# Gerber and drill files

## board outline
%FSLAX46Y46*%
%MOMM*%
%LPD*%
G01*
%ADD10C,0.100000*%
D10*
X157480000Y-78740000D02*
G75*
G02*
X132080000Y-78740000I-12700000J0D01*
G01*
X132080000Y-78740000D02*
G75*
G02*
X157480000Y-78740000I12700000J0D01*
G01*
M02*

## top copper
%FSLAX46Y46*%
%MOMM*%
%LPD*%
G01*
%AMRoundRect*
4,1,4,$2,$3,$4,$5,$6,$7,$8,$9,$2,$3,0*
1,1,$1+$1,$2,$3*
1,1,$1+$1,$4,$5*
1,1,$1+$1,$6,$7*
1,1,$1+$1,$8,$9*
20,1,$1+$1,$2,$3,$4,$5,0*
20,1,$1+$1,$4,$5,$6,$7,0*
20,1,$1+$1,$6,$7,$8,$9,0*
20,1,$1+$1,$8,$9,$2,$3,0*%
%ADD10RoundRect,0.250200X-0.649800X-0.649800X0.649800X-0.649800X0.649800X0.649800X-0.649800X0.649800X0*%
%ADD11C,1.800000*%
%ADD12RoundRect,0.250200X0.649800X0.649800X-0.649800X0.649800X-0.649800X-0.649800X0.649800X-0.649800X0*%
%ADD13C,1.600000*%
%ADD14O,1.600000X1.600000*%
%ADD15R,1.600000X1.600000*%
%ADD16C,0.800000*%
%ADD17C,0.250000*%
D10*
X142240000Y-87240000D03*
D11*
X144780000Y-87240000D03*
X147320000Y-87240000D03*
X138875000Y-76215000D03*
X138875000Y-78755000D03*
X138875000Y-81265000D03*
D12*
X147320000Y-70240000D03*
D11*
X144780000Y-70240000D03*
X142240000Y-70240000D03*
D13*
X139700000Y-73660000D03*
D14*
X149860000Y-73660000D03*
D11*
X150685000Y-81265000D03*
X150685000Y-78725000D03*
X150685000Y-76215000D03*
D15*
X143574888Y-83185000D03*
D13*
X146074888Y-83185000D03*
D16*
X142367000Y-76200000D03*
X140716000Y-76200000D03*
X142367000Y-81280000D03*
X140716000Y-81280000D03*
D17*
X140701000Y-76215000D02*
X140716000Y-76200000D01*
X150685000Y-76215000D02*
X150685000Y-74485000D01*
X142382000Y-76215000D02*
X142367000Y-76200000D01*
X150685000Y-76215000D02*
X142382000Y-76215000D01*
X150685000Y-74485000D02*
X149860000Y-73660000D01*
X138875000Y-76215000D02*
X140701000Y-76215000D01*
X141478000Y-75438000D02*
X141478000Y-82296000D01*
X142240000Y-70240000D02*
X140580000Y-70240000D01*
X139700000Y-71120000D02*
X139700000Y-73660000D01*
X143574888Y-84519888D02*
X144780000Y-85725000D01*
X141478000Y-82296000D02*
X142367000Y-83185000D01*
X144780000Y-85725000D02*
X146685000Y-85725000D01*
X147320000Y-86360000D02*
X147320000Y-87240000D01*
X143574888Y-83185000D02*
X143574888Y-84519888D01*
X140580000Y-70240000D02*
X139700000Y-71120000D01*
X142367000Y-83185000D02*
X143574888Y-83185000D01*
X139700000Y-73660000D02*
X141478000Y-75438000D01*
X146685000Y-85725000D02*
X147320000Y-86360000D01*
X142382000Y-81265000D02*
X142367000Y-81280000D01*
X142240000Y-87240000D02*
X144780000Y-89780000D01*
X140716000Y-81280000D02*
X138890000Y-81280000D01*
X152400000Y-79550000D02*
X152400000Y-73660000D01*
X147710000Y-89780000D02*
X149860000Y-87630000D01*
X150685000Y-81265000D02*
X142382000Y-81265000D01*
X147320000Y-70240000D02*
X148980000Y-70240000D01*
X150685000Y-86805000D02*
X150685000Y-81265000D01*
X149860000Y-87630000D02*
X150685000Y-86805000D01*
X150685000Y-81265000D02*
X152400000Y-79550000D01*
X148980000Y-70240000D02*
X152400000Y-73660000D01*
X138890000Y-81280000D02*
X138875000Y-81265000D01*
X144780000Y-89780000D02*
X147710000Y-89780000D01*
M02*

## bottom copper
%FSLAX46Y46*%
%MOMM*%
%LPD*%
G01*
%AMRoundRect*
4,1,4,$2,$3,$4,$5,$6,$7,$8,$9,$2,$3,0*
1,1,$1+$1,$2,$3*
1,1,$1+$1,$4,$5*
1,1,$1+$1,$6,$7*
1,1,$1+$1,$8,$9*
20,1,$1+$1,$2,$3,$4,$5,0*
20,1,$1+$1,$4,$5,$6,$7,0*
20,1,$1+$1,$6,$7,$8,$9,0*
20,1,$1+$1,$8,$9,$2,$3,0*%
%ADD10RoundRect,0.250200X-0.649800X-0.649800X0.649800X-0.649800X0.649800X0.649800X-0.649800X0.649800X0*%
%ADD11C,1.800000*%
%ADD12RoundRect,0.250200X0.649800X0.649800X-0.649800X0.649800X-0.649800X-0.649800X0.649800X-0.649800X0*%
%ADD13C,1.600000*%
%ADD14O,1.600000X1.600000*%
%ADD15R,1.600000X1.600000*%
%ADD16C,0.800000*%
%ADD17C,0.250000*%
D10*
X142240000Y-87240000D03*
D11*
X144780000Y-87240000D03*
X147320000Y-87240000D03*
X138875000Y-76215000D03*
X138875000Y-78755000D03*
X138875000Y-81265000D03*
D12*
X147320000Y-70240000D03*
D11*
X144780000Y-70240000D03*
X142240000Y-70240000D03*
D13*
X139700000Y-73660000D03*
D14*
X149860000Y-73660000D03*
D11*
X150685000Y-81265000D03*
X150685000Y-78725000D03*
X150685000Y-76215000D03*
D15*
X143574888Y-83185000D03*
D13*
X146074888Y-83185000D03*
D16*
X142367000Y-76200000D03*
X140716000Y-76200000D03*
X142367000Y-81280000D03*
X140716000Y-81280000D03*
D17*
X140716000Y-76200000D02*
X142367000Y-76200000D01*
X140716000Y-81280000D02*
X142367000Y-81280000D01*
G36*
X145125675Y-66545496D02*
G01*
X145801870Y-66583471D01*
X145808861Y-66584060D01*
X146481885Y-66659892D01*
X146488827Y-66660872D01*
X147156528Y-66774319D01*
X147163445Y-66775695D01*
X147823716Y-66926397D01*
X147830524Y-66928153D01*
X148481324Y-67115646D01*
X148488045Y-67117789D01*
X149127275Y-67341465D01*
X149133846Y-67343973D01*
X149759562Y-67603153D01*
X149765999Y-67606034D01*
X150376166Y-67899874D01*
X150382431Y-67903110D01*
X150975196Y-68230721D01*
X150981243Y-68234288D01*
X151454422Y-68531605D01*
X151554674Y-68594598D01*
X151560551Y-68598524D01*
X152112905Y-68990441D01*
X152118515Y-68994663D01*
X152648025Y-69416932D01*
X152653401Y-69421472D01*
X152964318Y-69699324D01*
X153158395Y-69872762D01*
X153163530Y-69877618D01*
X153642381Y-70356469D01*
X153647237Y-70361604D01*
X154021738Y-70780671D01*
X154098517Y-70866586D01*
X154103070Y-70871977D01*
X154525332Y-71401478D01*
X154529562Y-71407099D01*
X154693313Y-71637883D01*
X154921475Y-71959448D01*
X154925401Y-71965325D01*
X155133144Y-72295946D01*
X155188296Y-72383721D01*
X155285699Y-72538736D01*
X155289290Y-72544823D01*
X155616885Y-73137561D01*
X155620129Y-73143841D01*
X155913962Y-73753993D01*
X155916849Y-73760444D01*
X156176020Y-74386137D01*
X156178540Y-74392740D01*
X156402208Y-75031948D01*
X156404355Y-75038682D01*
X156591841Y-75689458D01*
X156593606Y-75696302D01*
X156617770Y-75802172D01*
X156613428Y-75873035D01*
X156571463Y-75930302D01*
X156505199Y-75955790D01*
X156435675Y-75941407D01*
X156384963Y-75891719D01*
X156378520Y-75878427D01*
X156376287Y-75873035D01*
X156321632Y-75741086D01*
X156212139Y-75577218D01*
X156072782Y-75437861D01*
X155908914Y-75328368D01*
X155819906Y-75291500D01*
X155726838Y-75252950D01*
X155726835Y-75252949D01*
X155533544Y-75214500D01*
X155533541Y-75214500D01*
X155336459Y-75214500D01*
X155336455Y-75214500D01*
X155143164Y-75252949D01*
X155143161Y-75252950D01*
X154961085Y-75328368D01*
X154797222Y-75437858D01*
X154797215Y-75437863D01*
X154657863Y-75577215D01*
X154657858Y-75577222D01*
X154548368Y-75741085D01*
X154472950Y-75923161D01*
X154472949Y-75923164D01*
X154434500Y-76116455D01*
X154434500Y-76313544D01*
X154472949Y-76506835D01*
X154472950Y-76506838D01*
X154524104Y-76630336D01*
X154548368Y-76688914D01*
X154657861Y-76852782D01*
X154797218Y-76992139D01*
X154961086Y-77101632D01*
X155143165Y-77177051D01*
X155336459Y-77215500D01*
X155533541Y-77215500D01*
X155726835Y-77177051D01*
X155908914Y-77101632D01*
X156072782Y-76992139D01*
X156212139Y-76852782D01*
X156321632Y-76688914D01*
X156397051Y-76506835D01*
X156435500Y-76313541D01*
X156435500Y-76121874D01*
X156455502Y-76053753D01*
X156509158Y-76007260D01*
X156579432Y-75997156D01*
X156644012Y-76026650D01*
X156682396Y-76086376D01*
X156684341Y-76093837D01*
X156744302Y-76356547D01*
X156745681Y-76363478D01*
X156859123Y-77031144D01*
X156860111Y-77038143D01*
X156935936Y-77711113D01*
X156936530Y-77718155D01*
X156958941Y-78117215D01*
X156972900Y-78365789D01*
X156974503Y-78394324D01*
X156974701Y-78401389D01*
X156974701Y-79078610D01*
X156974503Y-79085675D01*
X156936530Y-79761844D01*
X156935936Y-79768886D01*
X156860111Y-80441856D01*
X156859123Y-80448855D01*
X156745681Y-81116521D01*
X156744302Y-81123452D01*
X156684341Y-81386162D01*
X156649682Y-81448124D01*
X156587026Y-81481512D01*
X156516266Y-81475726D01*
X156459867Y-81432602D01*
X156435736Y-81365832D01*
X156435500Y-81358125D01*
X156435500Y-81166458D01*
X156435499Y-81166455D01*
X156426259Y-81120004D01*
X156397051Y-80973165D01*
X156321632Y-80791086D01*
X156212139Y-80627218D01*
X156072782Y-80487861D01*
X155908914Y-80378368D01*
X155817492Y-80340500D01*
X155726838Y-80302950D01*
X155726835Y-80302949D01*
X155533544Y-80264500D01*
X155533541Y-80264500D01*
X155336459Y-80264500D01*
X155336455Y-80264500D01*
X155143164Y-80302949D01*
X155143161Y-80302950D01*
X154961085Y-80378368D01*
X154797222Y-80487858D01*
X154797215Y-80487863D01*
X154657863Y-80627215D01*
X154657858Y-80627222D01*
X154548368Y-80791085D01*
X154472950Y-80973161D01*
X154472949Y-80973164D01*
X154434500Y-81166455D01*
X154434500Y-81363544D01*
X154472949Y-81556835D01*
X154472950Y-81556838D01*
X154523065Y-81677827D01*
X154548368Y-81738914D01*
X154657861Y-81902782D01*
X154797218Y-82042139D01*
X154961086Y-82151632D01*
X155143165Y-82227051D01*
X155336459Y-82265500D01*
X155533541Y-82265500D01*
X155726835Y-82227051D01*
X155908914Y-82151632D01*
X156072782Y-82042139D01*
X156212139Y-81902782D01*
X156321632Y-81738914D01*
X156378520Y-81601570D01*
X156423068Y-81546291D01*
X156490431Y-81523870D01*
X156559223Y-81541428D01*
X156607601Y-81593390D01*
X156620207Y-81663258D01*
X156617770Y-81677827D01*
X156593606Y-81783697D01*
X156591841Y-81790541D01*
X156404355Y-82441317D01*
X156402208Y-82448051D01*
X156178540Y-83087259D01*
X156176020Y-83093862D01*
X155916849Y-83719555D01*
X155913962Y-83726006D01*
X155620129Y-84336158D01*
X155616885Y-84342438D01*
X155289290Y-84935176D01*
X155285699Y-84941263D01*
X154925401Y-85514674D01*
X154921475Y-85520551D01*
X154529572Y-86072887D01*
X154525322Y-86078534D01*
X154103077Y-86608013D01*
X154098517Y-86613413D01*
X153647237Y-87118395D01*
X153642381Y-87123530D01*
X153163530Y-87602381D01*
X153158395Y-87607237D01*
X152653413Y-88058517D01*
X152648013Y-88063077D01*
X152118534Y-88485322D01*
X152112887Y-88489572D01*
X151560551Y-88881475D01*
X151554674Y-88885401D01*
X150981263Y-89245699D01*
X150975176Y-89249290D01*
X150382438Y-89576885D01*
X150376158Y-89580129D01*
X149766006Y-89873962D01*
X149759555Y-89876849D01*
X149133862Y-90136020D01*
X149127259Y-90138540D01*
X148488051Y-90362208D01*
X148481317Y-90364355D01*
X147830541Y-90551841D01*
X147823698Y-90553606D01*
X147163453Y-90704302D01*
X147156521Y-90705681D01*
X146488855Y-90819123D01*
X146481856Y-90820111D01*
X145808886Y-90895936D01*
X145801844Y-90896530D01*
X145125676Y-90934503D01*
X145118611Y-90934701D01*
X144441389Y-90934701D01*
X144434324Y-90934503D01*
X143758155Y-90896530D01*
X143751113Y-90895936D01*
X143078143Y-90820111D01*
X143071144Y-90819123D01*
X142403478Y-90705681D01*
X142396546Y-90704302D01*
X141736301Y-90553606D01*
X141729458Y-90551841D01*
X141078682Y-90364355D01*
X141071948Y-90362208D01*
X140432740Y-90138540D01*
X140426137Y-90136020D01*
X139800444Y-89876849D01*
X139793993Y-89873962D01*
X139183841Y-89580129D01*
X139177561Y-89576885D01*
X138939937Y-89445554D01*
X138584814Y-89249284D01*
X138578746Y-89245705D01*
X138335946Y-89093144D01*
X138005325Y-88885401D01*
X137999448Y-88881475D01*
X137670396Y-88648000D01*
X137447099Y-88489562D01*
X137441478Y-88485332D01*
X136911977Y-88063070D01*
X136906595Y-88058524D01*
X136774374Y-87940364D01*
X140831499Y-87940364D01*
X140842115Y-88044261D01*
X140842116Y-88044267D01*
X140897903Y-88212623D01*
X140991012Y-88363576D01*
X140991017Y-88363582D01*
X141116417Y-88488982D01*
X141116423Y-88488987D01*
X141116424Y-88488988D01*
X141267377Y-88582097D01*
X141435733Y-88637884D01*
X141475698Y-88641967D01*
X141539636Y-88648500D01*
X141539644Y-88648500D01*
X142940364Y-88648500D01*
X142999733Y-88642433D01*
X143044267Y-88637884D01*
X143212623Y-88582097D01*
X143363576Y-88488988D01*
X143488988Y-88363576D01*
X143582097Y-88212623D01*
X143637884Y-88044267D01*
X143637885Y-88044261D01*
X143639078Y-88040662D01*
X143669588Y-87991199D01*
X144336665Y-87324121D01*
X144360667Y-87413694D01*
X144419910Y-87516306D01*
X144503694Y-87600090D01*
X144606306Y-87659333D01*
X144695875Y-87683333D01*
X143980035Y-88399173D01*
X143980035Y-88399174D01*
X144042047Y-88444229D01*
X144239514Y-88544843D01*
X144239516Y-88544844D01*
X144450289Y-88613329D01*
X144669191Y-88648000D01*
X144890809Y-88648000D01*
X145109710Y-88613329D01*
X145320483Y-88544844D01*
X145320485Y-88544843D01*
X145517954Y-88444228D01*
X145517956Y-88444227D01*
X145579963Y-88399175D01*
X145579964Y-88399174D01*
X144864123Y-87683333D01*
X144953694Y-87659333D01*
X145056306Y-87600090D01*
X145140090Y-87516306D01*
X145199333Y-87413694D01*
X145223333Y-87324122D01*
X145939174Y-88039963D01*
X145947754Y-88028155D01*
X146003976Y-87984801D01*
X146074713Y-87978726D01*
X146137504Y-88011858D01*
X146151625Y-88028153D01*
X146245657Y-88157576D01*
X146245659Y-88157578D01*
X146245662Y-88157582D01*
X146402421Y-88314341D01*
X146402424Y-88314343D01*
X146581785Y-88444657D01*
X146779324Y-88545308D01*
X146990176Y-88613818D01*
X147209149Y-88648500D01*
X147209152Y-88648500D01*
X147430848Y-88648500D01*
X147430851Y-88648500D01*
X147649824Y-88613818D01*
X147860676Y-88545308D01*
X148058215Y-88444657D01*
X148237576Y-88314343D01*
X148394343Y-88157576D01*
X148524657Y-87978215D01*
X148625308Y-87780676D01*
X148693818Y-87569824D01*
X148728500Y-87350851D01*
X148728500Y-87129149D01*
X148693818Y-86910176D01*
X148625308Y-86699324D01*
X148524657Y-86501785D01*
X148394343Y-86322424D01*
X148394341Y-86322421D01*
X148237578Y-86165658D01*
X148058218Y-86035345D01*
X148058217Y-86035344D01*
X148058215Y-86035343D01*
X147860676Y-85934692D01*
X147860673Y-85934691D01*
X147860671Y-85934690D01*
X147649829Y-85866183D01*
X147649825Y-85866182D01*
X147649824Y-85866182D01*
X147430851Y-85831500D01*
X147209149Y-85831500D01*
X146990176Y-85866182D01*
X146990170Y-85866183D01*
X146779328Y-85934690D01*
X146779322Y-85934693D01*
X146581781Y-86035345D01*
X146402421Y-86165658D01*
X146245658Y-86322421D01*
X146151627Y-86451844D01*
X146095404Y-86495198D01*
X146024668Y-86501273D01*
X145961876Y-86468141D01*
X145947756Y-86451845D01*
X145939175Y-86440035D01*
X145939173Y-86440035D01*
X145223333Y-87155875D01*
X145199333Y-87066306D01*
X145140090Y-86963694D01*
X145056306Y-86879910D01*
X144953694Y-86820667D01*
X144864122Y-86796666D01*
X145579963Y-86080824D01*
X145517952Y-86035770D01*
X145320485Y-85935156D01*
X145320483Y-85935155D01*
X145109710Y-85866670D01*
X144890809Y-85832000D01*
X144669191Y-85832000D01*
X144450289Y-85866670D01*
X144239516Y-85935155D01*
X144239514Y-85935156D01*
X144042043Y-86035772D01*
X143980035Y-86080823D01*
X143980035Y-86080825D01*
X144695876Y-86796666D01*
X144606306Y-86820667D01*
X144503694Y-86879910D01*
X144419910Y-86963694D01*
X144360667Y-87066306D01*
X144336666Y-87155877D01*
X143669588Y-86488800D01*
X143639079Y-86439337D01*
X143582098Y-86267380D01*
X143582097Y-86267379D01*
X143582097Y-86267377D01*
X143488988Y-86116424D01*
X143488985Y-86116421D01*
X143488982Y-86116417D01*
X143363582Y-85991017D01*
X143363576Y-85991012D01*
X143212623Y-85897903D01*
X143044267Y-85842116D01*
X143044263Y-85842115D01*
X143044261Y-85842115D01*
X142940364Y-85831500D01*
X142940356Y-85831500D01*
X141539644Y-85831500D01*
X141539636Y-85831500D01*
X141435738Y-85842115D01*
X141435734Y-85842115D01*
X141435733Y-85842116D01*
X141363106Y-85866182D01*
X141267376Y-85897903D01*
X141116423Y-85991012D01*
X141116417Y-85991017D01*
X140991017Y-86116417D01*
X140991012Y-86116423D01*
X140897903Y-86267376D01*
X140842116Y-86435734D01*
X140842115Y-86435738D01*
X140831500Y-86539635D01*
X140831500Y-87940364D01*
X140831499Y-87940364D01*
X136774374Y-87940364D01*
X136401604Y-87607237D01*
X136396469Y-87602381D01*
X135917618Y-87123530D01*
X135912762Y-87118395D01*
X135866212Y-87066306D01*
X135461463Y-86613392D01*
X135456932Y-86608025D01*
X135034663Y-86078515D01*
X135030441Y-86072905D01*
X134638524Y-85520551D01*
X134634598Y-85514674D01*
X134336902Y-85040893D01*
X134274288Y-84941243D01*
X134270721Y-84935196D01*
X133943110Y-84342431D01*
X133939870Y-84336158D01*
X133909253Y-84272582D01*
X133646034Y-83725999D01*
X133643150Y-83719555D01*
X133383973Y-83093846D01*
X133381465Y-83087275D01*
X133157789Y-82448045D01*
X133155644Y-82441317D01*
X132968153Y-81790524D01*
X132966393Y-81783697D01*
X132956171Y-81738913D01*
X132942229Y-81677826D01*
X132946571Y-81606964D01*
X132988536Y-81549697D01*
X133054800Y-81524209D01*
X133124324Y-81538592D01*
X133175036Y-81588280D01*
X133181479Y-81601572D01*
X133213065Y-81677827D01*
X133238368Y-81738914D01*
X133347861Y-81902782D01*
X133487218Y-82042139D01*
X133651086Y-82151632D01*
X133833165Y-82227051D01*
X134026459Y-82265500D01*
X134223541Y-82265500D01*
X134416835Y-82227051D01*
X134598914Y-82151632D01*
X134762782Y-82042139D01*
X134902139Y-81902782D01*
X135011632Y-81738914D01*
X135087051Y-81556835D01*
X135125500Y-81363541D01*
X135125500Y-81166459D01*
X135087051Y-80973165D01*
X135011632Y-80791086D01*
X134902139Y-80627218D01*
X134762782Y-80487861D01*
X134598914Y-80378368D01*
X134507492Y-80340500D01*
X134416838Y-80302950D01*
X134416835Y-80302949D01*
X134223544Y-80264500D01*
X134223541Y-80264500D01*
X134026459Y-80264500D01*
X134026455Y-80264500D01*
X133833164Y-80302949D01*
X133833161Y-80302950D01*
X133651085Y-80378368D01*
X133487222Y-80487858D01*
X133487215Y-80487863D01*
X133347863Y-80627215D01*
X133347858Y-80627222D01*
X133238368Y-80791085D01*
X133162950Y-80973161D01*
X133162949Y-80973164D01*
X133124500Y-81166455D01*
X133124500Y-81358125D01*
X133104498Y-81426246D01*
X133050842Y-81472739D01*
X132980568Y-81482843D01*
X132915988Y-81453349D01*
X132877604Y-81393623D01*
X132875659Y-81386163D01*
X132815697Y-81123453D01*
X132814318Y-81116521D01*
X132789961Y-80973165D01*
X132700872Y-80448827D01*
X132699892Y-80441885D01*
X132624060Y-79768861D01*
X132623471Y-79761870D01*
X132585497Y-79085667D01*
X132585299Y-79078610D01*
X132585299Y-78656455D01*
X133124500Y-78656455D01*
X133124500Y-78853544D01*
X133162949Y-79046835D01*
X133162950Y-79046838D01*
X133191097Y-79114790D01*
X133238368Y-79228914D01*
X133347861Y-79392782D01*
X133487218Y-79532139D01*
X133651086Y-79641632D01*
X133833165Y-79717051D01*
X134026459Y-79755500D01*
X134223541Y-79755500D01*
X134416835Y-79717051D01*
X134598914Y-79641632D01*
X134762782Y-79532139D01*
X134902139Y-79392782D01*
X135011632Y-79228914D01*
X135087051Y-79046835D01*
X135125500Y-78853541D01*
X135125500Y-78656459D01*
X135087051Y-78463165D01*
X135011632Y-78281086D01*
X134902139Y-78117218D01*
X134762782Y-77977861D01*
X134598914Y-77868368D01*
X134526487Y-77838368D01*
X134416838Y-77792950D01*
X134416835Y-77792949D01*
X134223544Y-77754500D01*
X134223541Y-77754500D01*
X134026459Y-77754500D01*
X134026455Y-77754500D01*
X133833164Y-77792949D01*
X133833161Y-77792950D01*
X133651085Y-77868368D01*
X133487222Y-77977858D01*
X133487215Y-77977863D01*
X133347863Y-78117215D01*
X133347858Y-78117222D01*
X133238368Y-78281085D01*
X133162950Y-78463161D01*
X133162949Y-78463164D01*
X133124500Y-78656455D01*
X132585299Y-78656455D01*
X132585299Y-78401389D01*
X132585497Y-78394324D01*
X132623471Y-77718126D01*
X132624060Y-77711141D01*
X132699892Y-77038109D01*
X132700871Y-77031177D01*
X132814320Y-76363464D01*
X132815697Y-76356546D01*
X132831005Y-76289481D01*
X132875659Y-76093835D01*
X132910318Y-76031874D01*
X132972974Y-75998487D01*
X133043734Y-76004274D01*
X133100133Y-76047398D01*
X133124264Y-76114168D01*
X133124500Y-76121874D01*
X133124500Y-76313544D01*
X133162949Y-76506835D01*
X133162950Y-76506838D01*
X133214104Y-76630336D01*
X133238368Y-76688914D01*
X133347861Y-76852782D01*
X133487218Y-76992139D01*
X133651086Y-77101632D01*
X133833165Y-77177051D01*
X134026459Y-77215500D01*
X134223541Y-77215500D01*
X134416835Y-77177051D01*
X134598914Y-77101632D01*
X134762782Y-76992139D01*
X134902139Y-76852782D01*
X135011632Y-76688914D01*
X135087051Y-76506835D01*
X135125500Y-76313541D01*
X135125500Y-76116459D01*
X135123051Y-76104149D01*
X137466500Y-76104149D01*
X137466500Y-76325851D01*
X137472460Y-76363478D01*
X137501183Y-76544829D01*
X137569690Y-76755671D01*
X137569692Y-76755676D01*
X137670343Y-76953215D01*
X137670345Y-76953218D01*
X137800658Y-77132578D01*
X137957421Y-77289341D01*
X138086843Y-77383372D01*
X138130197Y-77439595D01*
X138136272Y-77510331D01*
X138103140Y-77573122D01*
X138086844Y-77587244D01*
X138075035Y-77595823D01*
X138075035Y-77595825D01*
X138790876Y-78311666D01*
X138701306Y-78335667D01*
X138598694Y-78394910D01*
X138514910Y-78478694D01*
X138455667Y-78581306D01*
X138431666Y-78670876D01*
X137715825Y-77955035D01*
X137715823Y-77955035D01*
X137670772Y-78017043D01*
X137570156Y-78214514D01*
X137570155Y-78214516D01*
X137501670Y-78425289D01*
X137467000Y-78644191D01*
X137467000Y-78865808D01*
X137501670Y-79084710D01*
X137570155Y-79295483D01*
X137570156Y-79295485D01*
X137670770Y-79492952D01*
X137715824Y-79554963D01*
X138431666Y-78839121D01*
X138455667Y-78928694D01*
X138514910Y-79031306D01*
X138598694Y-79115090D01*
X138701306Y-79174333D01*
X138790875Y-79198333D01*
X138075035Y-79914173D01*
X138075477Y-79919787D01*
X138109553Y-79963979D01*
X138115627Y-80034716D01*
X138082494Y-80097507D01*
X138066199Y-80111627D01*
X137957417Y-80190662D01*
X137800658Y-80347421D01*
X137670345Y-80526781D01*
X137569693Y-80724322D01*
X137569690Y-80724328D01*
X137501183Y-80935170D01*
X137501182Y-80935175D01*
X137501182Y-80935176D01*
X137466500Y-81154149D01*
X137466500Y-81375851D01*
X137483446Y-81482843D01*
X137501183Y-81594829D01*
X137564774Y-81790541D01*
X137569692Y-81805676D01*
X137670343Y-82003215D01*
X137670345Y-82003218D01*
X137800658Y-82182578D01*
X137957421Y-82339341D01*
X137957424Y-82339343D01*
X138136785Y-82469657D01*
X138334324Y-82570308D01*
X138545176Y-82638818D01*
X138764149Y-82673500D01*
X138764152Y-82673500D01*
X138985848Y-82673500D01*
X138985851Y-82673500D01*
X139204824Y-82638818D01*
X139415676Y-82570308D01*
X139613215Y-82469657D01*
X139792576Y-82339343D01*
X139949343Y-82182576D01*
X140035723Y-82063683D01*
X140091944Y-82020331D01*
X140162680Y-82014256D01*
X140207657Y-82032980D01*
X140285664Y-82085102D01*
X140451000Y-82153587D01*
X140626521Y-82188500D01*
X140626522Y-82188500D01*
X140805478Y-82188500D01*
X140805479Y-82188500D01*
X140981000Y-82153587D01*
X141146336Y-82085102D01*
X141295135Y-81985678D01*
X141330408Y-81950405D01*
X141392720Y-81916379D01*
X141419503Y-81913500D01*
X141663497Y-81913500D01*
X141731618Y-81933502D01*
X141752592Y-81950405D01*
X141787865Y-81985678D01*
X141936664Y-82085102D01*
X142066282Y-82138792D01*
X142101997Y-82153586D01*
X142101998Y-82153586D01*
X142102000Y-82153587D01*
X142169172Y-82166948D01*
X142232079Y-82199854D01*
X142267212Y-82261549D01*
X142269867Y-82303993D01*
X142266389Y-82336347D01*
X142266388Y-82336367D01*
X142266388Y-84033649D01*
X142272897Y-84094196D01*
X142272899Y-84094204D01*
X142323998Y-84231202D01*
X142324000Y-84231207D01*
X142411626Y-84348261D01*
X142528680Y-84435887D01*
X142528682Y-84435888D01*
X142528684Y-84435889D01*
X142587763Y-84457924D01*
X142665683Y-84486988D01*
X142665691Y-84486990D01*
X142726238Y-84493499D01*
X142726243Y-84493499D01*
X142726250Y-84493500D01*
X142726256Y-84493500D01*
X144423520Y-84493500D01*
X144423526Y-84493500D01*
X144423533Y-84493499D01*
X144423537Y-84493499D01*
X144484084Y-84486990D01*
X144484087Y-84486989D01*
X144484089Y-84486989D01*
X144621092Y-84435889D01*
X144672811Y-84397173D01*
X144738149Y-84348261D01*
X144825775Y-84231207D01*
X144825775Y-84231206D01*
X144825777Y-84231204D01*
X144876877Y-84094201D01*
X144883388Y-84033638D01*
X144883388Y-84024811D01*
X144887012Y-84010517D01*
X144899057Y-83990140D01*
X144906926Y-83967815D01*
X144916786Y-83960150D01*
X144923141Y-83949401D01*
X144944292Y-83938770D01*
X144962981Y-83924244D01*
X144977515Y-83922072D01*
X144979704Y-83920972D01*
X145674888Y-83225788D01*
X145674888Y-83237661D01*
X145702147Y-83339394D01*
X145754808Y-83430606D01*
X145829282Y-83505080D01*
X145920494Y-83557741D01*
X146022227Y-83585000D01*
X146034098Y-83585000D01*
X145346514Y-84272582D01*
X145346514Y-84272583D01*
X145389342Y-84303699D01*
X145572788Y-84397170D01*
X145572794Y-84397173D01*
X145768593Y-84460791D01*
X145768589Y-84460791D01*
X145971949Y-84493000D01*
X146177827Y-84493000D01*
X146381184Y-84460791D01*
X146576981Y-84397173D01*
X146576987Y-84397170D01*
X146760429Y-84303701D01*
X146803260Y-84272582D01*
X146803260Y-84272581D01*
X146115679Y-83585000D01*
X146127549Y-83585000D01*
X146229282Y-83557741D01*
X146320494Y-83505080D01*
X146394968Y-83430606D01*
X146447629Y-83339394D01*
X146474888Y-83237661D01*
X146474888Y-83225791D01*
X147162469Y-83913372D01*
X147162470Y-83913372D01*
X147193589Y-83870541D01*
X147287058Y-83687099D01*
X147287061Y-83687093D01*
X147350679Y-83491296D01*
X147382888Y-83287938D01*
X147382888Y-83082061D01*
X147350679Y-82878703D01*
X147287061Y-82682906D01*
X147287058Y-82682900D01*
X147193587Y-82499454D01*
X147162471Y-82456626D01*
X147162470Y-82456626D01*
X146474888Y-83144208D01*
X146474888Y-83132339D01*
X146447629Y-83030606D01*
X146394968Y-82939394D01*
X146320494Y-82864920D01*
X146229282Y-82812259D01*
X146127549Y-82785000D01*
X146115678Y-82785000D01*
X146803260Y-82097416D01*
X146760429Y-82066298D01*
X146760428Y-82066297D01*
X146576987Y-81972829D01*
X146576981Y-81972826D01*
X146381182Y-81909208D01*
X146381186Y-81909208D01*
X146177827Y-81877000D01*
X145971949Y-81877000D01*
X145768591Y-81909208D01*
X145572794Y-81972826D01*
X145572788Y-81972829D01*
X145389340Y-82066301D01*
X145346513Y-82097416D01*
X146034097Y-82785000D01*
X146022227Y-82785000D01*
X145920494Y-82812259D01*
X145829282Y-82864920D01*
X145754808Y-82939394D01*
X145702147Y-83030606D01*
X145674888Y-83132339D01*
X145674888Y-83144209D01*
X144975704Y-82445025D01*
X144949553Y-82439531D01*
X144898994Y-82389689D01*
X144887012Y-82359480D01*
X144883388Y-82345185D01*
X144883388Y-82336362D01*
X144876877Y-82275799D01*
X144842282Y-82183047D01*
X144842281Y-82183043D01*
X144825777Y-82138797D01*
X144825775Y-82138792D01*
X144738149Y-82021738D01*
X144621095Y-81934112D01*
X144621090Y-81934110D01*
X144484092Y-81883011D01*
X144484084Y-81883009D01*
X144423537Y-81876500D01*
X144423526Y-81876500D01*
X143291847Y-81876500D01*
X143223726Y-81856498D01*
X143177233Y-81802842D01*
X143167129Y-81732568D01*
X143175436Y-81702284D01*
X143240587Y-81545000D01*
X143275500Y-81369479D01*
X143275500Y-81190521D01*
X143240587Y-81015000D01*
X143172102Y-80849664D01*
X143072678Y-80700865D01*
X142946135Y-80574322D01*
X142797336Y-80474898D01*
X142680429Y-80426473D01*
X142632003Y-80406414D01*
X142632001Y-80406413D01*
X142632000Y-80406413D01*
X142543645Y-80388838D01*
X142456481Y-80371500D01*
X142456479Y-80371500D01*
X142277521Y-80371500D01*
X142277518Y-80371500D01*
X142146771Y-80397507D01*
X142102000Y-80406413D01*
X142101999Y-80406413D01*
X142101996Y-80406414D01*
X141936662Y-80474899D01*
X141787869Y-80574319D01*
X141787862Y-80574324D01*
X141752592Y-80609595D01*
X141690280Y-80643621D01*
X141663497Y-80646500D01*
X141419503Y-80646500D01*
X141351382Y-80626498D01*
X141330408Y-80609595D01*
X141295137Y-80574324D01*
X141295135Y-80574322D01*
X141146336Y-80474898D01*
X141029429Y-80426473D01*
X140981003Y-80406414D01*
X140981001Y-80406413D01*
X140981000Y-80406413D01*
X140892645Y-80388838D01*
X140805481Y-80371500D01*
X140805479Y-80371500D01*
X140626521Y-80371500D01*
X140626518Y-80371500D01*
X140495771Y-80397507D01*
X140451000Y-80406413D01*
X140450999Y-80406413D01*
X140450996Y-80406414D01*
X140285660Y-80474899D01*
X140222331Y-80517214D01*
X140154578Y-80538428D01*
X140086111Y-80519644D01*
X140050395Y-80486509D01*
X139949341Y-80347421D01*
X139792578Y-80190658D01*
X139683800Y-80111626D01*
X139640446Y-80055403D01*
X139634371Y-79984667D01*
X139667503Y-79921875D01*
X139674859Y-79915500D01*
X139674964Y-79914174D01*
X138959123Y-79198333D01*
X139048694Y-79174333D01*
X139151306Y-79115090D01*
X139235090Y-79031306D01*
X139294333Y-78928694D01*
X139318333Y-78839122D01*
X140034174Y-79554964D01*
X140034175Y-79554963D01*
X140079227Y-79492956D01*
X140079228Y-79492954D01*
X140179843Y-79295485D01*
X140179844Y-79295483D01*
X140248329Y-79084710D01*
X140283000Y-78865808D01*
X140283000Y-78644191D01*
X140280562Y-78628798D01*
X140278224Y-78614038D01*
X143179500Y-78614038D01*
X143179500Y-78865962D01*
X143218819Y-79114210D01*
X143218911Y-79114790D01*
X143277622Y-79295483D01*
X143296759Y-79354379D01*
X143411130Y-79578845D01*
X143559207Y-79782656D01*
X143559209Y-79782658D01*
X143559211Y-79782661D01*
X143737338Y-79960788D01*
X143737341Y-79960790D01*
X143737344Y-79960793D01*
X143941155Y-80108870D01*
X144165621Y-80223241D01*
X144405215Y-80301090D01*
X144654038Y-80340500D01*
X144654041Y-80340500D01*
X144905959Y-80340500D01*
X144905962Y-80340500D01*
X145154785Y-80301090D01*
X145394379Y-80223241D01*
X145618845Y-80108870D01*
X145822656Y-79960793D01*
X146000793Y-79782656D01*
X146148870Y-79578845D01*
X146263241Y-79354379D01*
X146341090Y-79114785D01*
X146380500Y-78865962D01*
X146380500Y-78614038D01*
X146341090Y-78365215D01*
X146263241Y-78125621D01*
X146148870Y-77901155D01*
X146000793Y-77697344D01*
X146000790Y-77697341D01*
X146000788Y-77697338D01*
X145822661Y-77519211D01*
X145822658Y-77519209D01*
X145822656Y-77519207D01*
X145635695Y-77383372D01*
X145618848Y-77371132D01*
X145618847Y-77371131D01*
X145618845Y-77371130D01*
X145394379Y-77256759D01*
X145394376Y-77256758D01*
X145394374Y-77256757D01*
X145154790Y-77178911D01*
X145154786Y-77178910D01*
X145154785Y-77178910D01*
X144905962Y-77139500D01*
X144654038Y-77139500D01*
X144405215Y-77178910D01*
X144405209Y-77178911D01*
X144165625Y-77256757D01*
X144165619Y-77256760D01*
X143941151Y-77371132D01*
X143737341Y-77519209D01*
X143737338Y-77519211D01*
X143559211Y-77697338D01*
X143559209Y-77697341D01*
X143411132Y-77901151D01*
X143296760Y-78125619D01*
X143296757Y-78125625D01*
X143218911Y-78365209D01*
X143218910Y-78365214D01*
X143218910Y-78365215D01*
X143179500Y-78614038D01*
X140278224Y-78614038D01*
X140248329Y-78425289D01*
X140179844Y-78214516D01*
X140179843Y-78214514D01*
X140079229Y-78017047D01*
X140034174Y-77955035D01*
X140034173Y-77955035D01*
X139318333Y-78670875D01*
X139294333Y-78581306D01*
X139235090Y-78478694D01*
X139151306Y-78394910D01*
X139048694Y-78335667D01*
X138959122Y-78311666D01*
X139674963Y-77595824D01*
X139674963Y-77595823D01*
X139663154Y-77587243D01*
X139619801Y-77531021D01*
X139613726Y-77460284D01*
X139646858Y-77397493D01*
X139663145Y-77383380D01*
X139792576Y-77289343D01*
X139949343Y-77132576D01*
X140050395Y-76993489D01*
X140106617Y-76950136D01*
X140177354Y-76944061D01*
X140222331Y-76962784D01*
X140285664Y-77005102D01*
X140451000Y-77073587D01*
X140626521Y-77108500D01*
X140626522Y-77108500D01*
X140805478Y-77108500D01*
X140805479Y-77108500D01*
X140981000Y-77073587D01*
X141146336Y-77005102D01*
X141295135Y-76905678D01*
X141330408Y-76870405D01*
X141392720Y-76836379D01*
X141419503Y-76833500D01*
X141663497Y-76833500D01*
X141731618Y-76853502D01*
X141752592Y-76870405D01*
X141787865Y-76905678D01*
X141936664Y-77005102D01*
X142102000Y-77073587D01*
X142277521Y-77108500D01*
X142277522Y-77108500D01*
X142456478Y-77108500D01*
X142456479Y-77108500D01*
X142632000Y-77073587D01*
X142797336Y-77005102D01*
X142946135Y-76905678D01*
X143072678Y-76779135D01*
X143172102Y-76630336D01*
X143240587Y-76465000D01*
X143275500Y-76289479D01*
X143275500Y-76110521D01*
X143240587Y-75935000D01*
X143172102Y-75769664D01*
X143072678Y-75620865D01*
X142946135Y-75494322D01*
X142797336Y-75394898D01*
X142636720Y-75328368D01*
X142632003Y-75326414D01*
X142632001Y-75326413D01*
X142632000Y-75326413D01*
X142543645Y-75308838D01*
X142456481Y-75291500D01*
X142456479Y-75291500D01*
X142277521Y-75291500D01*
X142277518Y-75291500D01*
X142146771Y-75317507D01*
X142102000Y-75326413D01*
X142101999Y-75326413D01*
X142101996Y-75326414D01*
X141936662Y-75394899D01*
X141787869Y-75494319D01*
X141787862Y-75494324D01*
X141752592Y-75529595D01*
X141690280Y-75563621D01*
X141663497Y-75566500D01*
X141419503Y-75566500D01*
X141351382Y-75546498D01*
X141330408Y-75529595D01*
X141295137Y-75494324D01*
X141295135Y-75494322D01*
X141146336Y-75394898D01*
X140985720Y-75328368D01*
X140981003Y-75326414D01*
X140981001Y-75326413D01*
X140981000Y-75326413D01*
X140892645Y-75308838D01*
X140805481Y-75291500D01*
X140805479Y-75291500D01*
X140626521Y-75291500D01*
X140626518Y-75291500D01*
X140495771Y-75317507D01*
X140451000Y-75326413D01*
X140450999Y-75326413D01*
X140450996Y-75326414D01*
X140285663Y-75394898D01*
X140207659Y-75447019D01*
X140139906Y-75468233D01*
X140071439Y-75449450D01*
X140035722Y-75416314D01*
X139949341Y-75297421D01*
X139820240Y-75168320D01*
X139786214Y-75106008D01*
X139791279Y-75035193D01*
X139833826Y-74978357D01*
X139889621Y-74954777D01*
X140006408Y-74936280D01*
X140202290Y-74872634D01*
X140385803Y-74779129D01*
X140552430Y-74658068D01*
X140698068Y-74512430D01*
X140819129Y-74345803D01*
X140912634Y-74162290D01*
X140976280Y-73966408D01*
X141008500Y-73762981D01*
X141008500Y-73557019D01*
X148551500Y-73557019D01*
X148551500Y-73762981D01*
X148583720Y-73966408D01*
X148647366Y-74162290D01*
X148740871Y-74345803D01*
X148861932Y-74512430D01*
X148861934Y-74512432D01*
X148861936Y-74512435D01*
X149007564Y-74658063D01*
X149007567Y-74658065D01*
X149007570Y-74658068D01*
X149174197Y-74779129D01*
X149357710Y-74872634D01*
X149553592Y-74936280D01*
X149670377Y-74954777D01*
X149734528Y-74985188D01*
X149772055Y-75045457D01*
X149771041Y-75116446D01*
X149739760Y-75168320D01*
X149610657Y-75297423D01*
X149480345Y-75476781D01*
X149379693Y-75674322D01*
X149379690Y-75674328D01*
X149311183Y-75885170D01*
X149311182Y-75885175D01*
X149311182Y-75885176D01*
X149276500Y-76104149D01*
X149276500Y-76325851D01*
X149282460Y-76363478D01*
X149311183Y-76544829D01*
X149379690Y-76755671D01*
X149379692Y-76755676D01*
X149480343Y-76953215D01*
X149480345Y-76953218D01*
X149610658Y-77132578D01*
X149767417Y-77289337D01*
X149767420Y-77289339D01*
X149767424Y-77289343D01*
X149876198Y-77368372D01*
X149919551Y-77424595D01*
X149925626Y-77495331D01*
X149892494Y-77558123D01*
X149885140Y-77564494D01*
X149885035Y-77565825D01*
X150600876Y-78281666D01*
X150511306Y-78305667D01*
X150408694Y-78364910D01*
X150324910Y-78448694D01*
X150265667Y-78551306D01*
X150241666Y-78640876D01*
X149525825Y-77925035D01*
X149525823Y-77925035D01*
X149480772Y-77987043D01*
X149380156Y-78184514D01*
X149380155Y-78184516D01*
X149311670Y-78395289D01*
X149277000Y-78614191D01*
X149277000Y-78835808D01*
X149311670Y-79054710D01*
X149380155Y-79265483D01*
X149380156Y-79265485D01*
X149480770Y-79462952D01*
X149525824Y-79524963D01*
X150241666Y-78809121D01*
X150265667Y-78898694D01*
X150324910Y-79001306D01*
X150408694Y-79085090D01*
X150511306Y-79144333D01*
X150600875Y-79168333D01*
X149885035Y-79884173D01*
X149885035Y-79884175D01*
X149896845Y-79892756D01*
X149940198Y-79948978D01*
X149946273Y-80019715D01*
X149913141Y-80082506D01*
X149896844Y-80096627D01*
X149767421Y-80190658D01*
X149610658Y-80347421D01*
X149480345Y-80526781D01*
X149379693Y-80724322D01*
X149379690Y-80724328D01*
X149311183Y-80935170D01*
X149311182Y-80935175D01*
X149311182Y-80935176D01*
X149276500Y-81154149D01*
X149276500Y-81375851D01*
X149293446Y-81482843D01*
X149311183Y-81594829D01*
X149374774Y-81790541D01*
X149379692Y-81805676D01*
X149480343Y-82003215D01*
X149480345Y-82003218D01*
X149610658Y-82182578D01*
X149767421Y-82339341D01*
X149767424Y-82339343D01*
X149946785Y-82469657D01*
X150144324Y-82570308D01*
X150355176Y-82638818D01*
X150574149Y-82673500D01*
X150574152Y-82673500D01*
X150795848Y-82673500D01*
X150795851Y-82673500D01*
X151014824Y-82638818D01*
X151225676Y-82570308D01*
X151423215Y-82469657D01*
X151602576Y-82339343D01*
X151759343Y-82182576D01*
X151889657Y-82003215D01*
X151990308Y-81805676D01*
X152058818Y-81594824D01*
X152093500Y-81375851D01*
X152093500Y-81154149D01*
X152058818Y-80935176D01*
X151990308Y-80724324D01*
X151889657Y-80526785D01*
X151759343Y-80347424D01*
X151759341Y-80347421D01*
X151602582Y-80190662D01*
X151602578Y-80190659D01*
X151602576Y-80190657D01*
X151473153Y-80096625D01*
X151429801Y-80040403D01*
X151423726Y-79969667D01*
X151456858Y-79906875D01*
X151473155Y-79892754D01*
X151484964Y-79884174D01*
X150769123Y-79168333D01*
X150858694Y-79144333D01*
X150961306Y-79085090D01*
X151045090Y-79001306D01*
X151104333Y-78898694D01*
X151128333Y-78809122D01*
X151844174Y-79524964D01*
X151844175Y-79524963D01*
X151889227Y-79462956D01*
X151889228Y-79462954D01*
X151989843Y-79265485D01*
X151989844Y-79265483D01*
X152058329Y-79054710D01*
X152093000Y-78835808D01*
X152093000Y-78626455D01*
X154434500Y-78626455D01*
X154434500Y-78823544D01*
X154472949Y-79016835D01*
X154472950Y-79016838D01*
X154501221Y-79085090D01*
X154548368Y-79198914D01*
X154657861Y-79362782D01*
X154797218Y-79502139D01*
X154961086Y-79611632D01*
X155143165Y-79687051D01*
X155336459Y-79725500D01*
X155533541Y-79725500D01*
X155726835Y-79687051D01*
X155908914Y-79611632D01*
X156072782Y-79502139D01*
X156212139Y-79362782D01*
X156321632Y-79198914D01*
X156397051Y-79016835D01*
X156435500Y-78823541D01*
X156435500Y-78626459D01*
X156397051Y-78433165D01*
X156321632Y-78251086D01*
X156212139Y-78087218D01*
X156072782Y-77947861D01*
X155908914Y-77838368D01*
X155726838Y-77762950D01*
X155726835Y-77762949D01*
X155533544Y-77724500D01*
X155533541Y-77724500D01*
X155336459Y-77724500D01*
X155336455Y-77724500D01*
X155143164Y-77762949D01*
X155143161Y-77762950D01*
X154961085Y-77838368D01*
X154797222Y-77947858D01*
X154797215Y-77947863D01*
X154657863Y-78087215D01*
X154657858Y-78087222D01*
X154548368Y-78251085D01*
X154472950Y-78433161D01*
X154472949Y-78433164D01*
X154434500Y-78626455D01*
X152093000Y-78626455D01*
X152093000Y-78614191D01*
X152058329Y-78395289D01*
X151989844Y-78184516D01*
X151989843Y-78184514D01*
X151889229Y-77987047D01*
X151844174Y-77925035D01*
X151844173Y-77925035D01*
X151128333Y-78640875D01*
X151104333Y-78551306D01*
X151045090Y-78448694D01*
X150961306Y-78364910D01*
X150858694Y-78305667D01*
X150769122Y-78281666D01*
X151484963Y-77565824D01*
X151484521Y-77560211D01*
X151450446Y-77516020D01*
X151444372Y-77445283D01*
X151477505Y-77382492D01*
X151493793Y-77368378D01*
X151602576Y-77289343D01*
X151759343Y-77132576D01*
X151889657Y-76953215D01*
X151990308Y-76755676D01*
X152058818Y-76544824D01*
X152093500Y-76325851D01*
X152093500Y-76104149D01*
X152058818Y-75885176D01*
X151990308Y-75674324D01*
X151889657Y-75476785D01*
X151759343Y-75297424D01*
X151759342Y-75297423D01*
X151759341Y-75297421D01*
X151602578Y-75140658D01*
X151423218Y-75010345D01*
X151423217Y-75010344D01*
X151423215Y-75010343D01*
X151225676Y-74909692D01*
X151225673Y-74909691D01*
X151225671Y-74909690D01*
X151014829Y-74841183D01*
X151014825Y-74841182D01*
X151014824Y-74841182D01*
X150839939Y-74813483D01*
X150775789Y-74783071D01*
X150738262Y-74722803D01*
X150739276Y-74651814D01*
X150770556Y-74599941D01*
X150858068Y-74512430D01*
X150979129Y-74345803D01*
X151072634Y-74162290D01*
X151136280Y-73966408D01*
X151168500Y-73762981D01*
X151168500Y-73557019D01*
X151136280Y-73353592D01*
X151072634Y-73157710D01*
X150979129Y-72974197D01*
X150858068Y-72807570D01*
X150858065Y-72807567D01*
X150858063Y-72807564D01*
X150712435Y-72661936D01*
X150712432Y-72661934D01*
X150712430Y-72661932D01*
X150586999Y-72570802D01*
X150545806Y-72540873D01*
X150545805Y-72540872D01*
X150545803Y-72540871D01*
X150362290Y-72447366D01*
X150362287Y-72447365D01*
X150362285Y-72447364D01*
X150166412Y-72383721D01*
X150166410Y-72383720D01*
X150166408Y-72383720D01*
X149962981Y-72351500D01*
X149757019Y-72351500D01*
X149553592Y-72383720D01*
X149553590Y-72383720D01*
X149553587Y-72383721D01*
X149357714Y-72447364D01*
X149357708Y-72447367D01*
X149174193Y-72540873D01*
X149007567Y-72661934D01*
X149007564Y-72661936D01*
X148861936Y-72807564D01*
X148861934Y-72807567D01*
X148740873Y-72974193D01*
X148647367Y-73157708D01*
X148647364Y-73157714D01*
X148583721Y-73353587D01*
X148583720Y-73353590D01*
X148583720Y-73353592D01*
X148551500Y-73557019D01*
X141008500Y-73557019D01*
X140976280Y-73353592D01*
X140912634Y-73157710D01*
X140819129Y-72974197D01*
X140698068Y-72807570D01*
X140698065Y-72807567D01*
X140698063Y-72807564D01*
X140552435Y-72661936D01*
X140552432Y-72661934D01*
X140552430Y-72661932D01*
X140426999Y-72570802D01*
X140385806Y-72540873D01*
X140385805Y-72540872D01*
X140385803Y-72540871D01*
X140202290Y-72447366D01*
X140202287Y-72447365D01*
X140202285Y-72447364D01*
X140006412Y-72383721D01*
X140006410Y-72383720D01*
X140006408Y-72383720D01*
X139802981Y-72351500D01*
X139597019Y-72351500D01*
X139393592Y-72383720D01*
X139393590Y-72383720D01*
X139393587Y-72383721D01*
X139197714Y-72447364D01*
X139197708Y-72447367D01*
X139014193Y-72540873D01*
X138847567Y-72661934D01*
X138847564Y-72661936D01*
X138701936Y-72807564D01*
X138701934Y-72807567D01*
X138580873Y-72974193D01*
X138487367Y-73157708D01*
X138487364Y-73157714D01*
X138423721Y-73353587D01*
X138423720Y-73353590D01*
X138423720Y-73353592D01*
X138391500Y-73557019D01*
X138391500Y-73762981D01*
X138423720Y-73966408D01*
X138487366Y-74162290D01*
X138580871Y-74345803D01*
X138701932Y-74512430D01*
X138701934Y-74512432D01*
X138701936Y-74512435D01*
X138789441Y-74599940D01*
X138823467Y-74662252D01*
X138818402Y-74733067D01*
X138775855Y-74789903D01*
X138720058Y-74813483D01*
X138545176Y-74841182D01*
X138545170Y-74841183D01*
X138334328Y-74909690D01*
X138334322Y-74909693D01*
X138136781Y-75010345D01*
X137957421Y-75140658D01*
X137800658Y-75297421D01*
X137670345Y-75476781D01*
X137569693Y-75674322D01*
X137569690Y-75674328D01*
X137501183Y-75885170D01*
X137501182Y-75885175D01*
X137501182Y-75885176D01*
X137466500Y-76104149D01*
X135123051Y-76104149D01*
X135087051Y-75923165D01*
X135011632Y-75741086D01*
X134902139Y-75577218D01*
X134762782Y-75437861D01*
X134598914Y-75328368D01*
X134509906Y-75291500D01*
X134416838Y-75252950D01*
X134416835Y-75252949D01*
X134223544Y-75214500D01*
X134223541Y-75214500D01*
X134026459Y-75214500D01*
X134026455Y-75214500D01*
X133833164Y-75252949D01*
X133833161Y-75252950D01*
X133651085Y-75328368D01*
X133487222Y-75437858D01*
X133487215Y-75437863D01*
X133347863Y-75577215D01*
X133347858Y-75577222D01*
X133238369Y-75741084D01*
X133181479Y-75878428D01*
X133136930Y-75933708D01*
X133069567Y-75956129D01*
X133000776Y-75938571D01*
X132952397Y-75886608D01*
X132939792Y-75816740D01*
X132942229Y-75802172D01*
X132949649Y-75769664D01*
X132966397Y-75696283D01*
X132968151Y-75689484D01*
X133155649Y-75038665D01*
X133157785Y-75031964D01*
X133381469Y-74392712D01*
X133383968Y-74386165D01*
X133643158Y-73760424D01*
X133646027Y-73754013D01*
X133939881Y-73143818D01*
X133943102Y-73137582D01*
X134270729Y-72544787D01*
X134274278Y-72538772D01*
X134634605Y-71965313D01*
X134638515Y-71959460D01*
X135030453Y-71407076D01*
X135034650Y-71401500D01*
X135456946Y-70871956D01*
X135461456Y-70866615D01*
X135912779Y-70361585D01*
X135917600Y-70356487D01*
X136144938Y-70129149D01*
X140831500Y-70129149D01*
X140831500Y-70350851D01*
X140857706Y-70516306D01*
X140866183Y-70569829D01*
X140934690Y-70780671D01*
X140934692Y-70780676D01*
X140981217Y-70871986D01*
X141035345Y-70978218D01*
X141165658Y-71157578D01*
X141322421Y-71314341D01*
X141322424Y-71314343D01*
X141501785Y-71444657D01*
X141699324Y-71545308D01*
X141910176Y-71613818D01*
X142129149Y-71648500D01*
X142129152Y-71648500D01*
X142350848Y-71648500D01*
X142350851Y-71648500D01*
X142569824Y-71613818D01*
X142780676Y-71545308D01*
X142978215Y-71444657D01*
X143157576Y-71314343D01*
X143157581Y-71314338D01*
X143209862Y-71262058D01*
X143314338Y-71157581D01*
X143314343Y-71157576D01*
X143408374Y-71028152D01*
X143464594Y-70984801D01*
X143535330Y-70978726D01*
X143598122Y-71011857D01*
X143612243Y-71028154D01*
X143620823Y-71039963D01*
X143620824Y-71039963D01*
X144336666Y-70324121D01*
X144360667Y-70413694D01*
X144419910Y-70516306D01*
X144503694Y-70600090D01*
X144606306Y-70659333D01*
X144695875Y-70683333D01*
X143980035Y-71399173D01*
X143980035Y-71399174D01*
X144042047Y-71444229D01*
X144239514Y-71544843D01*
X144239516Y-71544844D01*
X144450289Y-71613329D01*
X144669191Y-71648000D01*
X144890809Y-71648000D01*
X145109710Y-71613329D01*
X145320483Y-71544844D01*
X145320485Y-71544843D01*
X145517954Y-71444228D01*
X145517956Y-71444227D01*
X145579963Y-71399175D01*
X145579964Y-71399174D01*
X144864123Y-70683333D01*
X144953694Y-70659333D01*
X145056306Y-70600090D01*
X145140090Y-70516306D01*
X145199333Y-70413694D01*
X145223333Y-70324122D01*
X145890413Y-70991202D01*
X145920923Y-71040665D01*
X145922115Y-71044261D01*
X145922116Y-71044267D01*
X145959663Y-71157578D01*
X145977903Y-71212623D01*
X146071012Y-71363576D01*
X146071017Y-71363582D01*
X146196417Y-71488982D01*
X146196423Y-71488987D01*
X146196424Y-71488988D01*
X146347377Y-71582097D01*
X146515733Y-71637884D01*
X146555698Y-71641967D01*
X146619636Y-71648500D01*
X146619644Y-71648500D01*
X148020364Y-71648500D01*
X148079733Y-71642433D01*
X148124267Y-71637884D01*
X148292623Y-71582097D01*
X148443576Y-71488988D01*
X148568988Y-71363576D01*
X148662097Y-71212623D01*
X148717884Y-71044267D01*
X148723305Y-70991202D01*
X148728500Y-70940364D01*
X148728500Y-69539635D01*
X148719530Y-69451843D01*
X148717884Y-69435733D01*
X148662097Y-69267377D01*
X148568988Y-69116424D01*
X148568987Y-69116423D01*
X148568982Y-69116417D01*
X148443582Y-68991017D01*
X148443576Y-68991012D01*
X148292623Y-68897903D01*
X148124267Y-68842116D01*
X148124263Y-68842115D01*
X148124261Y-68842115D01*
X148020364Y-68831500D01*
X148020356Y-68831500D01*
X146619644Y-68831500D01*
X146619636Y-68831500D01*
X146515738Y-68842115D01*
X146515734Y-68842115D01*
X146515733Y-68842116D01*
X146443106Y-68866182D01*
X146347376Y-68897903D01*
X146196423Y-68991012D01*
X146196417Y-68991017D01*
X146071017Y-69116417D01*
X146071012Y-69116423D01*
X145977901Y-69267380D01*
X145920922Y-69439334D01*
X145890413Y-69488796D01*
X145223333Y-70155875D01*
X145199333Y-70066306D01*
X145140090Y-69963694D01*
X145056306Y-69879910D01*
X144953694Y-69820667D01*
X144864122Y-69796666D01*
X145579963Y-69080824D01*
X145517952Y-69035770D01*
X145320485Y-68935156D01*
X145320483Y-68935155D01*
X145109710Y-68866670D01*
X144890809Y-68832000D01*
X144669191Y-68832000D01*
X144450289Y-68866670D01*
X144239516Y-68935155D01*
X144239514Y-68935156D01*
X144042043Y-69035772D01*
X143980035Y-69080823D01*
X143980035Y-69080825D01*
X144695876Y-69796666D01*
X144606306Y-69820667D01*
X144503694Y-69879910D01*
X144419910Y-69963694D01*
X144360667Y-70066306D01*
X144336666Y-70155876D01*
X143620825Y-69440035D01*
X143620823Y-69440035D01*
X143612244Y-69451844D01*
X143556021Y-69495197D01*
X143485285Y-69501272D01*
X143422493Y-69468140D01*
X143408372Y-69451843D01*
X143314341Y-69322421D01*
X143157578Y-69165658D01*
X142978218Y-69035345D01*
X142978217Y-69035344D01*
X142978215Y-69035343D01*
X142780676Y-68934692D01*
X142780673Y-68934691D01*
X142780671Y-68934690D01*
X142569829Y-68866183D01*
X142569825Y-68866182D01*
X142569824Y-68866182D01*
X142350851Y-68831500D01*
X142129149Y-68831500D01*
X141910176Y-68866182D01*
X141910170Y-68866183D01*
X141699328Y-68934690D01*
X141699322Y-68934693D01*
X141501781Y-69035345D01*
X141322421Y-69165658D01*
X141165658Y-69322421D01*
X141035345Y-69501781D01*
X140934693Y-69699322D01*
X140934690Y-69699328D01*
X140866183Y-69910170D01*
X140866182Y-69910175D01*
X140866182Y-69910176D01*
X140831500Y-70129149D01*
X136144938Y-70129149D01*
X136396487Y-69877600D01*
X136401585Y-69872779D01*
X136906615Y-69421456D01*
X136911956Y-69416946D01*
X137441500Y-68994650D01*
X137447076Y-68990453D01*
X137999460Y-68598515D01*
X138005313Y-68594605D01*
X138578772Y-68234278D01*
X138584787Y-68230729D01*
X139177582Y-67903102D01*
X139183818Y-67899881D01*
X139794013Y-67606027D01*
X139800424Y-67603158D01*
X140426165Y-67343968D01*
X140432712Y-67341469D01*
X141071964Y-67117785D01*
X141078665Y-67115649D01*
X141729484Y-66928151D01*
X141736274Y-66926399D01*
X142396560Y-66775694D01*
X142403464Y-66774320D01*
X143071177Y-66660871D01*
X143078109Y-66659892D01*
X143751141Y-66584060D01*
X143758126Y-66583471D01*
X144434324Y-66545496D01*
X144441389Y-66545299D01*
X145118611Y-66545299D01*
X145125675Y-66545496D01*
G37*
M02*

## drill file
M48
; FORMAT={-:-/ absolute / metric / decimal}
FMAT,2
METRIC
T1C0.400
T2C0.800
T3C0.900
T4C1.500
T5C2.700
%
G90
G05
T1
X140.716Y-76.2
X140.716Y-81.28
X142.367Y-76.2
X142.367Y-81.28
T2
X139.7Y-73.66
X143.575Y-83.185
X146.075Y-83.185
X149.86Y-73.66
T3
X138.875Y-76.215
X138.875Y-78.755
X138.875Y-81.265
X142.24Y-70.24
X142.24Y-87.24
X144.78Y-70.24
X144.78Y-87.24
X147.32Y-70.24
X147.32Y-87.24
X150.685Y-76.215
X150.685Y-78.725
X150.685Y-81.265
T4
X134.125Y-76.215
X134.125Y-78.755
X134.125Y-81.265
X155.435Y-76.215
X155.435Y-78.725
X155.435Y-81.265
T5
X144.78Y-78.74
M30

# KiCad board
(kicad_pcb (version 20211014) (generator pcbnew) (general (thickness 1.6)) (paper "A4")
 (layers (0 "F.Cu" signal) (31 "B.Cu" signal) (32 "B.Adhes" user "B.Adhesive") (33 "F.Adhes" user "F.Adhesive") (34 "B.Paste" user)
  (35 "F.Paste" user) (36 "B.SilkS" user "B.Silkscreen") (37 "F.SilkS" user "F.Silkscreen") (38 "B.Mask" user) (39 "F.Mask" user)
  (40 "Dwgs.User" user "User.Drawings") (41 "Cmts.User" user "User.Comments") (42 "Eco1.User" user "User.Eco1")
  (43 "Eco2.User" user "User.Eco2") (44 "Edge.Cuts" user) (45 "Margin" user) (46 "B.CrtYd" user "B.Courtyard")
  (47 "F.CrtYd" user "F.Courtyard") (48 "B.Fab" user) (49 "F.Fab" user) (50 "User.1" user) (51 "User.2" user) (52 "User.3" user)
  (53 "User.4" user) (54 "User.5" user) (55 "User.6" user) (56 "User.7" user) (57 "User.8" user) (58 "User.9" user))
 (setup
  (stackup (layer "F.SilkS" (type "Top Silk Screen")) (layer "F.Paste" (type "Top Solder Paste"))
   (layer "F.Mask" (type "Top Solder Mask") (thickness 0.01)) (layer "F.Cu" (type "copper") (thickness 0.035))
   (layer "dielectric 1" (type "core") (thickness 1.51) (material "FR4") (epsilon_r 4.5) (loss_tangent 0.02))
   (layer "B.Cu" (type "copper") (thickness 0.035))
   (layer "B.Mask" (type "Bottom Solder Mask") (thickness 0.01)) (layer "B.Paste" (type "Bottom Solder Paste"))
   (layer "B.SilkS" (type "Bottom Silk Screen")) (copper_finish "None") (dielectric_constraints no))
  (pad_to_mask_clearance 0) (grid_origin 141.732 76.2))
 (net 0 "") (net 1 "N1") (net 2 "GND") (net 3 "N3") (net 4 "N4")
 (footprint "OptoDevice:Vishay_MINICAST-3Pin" (layer "F.Cu") (at 142.24 87.24)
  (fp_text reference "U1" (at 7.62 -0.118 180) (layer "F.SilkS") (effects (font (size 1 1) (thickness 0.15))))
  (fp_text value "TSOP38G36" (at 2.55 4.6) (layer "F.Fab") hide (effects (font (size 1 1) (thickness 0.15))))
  (pad "1" thru_hole roundrect (at 0 0) (size 1.8 1.8) (drill 0.9) (layers *.Cu *.Mask) (roundrect_rratio 0.139) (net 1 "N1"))
  (pad "2" thru_hole circle (at 2.54 0) (size 1.8 1.8) (drill 0.9) (layers *.Cu *.Mask) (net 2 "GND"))
  (pad "3" thru_hole circle (at 5.08 0) (size 1.8 1.8) (drill 0.9) (layers *.Cu *.Mask) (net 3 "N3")))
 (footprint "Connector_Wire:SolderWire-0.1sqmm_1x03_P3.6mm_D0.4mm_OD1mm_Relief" (layer "F.Cu") (at 138.875 75.155 -90)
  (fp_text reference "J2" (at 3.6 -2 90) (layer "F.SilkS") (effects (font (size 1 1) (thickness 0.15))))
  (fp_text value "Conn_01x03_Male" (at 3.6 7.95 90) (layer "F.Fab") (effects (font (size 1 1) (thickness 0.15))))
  (pad "" np_thru_hole circle (at 6.11 4.75 270) (size 1.5 1.5) (drill 1.5) (layers *.Cu *.Mask))
  (pad "" np_thru_hole circle (at 3.6 4.75 270) (size 1.5 1.5) (drill 1.5) (layers *.Cu *.Mask))
  (pad "" np_thru_hole circle (at 1.06 4.75 270) (size 1.5 1.5) (drill 1.5) (layers *.Cu *.Mask))
  (pad "1" thru_hole circle (at 1.06 0 270) (size 1.8 1.8) (drill 0.9) (layers *.Cu *.Mask) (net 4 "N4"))
  (pad "2" thru_hole circle (at 3.6 0 270) (size 1.8 1.8) (drill 0.9) (layers *.Cu *.Mask) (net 2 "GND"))
  (pad "3" thru_hole circle (at 6.11 0 270) (size 1.8 1.8) (drill 0.9) (layers *.Cu *.Mask) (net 1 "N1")))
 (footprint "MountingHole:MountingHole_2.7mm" (layer "F.Cu") (at 144.78 78.74)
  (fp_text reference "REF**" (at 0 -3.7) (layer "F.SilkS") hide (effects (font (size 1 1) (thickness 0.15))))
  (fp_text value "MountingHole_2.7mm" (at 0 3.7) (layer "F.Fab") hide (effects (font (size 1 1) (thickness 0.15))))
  (pad "" np_thru_hole circle (at 0 0) (size 2.7 2.7) (drill 2.7) (layers *.Cu *.Mask)))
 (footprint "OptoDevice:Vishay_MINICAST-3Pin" (layer "F.Cu") (at 147.32 70.24 180)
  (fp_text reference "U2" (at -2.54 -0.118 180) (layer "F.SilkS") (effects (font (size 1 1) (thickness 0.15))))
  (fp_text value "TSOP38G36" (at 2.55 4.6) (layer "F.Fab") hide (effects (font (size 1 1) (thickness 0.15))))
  (pad "1" thru_hole roundrect (at 0 0 180) (size 1.8 1.8) (drill 0.9) (layers *.Cu *.Mask) (roundrect_rratio 0.139) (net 1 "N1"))
  (pad "2" thru_hole circle (at 2.54 0 180) (size 1.8 1.8) (drill 0.9) (layers *.Cu *.Mask) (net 2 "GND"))
  (pad "3" thru_hole circle (at 5.08 0 180) (size 1.8 1.8) (drill 0.9) (layers *.Cu *.Mask) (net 3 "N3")))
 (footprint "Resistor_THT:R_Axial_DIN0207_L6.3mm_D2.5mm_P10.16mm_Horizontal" (layer "F.Cu") (at 139.7 73.66)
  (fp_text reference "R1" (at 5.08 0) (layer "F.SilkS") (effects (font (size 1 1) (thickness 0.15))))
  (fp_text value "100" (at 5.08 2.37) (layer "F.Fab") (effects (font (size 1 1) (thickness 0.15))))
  (pad "1" thru_hole circle (at 0 0) (size 1.6 1.6) (drill 0.8) (layers *.Cu *.Mask) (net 3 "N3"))
  (pad "2" thru_hole oval (at 10.16 0) (size 1.6 1.6) (drill 0.8) (layers *.Cu *.Mask) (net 4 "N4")))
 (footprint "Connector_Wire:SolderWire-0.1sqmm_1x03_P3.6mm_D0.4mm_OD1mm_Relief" (layer "F.Cu") (at 150.685 81.265 90)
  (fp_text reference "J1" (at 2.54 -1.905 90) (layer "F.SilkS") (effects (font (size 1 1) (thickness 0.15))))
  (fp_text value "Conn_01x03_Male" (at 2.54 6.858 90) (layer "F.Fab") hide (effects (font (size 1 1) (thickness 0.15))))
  (pad "" np_thru_hole circle (at 0 4.75 90) (size 1.5 1.5) (drill 1.5) (layers *.Cu *.Mask))
  (pad "" np_thru_hole circle (at 2.54 4.75 90) (size 1.5 1.5) (drill 1.5) (layers *.Cu *.Mask))
  (pad "" np_thru_hole circle (at 5.05 4.75 90) (size 1.5 1.5) (drill 1.5) (layers *.Cu *.Mask))
  (pad "1" thru_hole circle (at 0 0 90) (size 1.8 1.8) (drill 0.9) (layers *.Cu *.Mask) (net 1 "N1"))
  (pad "2" thru_hole circle (at 2.54 0 90) (size 1.8 1.8) (drill 0.9) (layers *.Cu *.Mask) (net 2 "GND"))
  (pad "3" thru_hole circle (at 5.05 0 90) (size 1.8 1.8) (drill 0.9) (layers *.Cu *.Mask) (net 4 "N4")))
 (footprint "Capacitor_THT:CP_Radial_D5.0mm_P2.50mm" (layer "F.Cu") (at 143.574888 83.185)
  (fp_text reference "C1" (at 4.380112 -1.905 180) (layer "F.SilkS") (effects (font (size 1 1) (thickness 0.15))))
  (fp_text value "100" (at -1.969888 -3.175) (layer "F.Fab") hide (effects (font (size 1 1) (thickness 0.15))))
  (pad "1" thru_hole rect (at 0 0) (size 1.6 1.6) (drill 0.8) (layers *.Cu *.Mask) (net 3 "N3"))
  (pad "2" thru_hole circle (at 2.5 0) (size 1.6 1.6) (drill 0.8) (layers *.Cu *.Mask) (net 2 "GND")))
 (gr_circle (center 144.78 78.74) (end 157.48 78.74) (layer "Edge.Cuts") (width 0.1) (fill none))
 (segment (start 140.701 76.215) (end 140.716 76.2) (width 0.25) (layer "F.Cu") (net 4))
 (segment (start 150.685 76.215) (end 150.685 74.485) (width 0.25) (layer "F.Cu") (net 4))
 (segment (start 142.382 76.215) (end 142.367 76.2) (width 0.25) (layer "F.Cu") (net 4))
 (segment (start 150.685 76.215) (end 142.382 76.215) (width 0.25) (layer "F.Cu") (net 4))
 (segment (start 150.685 74.485) (end 149.86 73.66) (width 0.25) (layer "F.Cu") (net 4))
 (segment (start 138.875 76.215) (end 140.701 76.215) (width 0.25) (layer "F.Cu") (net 4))
 (via (at 142.367 76.2) (size 0.8) (drill 0.4) (layers "F.Cu" "B.Cu") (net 4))
 (via (at 140.716 76.2) (size 0.8) (drill 0.4) (layers "F.Cu" "B.Cu") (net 4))
 (segment (start 140.716 76.2) (end 142.367 76.2) (width 0.25) (layer "B.Cu") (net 4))
 (segment (start 141.478 75.438) (end 141.478 82.296) (width 0.25) (layer "F.Cu") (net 3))
 (segment (start 142.24 70.24) (end 140.58 70.24) (width 0.25) (layer "F.Cu") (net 3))
 (segment (start 139.7 71.12) (end 139.7 73.66) (width 0.25) (layer "F.Cu") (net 3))
 (segment (start 143.574888 84.519888) (end 144.78 85.725) (width 0.25) (layer "F.Cu") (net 3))
 (segment (start 141.478 82.296) (end 142.367 83.185) (width 0.25) (layer "F.Cu") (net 3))
 (segment (start 144.78 85.725) (end 146.685 85.725) (width 0.25) (layer "F.Cu") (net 3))
 (segment (start 147.32 86.36) (end 147.32 87.24) (width 0.25) (layer "F.Cu") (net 3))
 (segment (start 143.574888 83.185) (end 143.574888 84.519888) (width 0.25) (layer "F.Cu") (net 3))
 (segment (start 140.58 70.24) (end 139.7 71.12) (width 0.25) (layer "F.Cu") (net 3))
 (segment (start 142.367 83.185) (end 143.574888 83.185) (width 0.25) (layer "F.Cu") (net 3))
 (segment (start 139.7 73.66) (end 141.478 75.438) (width 0.25) (layer "F.Cu") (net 3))
 (segment (start 146.685 85.725) (end 147.32 86.36) (width 0.25) (layer "F.Cu") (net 3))
 (segment (start 142.382 81.265) (end 142.367 81.28) (width 0.25) (layer "F.Cu") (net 1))
 (segment (start 142.24 87.24) (end 144.78 89.78) (width 0.25) (layer "F.Cu") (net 1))
 (segment (start 140.716 81.28) (end 138.89 81.28) (width 0.25) (layer "F.Cu") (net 1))
 (segment (start 152.4 79.55) (end 152.4 73.66) (width 0.25) (layer "F.Cu") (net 1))
 (segment (start 147.71 89.78) (end 149.86 87.63) (width 0.25) (layer "F.Cu") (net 1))
 (segment (start 150.685 81.265) (end 142.382 81.265) (width 0.25) (layer "F.Cu") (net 1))
 (segment (start 147.32 70.24) (end 148.98 70.24) (width 0.25) (layer "F.Cu") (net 1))
 (segment (start 150.685 86.805) (end 150.685 81.265) (width 0.25) (layer "F.Cu") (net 1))
 (segment (start 149.86 87.63) (end 150.685 86.805) (width 0.25) (layer "F.Cu") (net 1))
 (segment (start 150.685 81.265) (end 152.4 79.55) (width 0.25) (layer "F.Cu") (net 1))
 (segment (start 148.98 70.24) (end 152.4 73.66) (width 0.25) (layer "F.Cu") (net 1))
 (segment (start 138.89 81.28) (end 138.875 81.265) (width 0.25) (layer "F.Cu") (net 1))
 (segment (start 144.78 89.78) (end 147.71 89.78) (width 0.25) (layer "F.Cu") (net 1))
 (via (at 142.367 81.28) (size 0.8) (drill 0.4) (layers "F.Cu" "B.Cu") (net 1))
 (via (at 140.716 81.28) (size 0.8) (drill 0.4) (layers "F.Cu" "B.Cu") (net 1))
 (segment (start 140.716 81.28) (end 142.367 81.28) (width 0.25) (layer "B.Cu") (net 1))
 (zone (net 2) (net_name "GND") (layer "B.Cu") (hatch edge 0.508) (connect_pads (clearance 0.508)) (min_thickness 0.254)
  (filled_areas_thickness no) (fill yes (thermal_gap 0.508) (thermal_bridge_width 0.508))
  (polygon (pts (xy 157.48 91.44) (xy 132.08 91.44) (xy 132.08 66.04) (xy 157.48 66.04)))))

